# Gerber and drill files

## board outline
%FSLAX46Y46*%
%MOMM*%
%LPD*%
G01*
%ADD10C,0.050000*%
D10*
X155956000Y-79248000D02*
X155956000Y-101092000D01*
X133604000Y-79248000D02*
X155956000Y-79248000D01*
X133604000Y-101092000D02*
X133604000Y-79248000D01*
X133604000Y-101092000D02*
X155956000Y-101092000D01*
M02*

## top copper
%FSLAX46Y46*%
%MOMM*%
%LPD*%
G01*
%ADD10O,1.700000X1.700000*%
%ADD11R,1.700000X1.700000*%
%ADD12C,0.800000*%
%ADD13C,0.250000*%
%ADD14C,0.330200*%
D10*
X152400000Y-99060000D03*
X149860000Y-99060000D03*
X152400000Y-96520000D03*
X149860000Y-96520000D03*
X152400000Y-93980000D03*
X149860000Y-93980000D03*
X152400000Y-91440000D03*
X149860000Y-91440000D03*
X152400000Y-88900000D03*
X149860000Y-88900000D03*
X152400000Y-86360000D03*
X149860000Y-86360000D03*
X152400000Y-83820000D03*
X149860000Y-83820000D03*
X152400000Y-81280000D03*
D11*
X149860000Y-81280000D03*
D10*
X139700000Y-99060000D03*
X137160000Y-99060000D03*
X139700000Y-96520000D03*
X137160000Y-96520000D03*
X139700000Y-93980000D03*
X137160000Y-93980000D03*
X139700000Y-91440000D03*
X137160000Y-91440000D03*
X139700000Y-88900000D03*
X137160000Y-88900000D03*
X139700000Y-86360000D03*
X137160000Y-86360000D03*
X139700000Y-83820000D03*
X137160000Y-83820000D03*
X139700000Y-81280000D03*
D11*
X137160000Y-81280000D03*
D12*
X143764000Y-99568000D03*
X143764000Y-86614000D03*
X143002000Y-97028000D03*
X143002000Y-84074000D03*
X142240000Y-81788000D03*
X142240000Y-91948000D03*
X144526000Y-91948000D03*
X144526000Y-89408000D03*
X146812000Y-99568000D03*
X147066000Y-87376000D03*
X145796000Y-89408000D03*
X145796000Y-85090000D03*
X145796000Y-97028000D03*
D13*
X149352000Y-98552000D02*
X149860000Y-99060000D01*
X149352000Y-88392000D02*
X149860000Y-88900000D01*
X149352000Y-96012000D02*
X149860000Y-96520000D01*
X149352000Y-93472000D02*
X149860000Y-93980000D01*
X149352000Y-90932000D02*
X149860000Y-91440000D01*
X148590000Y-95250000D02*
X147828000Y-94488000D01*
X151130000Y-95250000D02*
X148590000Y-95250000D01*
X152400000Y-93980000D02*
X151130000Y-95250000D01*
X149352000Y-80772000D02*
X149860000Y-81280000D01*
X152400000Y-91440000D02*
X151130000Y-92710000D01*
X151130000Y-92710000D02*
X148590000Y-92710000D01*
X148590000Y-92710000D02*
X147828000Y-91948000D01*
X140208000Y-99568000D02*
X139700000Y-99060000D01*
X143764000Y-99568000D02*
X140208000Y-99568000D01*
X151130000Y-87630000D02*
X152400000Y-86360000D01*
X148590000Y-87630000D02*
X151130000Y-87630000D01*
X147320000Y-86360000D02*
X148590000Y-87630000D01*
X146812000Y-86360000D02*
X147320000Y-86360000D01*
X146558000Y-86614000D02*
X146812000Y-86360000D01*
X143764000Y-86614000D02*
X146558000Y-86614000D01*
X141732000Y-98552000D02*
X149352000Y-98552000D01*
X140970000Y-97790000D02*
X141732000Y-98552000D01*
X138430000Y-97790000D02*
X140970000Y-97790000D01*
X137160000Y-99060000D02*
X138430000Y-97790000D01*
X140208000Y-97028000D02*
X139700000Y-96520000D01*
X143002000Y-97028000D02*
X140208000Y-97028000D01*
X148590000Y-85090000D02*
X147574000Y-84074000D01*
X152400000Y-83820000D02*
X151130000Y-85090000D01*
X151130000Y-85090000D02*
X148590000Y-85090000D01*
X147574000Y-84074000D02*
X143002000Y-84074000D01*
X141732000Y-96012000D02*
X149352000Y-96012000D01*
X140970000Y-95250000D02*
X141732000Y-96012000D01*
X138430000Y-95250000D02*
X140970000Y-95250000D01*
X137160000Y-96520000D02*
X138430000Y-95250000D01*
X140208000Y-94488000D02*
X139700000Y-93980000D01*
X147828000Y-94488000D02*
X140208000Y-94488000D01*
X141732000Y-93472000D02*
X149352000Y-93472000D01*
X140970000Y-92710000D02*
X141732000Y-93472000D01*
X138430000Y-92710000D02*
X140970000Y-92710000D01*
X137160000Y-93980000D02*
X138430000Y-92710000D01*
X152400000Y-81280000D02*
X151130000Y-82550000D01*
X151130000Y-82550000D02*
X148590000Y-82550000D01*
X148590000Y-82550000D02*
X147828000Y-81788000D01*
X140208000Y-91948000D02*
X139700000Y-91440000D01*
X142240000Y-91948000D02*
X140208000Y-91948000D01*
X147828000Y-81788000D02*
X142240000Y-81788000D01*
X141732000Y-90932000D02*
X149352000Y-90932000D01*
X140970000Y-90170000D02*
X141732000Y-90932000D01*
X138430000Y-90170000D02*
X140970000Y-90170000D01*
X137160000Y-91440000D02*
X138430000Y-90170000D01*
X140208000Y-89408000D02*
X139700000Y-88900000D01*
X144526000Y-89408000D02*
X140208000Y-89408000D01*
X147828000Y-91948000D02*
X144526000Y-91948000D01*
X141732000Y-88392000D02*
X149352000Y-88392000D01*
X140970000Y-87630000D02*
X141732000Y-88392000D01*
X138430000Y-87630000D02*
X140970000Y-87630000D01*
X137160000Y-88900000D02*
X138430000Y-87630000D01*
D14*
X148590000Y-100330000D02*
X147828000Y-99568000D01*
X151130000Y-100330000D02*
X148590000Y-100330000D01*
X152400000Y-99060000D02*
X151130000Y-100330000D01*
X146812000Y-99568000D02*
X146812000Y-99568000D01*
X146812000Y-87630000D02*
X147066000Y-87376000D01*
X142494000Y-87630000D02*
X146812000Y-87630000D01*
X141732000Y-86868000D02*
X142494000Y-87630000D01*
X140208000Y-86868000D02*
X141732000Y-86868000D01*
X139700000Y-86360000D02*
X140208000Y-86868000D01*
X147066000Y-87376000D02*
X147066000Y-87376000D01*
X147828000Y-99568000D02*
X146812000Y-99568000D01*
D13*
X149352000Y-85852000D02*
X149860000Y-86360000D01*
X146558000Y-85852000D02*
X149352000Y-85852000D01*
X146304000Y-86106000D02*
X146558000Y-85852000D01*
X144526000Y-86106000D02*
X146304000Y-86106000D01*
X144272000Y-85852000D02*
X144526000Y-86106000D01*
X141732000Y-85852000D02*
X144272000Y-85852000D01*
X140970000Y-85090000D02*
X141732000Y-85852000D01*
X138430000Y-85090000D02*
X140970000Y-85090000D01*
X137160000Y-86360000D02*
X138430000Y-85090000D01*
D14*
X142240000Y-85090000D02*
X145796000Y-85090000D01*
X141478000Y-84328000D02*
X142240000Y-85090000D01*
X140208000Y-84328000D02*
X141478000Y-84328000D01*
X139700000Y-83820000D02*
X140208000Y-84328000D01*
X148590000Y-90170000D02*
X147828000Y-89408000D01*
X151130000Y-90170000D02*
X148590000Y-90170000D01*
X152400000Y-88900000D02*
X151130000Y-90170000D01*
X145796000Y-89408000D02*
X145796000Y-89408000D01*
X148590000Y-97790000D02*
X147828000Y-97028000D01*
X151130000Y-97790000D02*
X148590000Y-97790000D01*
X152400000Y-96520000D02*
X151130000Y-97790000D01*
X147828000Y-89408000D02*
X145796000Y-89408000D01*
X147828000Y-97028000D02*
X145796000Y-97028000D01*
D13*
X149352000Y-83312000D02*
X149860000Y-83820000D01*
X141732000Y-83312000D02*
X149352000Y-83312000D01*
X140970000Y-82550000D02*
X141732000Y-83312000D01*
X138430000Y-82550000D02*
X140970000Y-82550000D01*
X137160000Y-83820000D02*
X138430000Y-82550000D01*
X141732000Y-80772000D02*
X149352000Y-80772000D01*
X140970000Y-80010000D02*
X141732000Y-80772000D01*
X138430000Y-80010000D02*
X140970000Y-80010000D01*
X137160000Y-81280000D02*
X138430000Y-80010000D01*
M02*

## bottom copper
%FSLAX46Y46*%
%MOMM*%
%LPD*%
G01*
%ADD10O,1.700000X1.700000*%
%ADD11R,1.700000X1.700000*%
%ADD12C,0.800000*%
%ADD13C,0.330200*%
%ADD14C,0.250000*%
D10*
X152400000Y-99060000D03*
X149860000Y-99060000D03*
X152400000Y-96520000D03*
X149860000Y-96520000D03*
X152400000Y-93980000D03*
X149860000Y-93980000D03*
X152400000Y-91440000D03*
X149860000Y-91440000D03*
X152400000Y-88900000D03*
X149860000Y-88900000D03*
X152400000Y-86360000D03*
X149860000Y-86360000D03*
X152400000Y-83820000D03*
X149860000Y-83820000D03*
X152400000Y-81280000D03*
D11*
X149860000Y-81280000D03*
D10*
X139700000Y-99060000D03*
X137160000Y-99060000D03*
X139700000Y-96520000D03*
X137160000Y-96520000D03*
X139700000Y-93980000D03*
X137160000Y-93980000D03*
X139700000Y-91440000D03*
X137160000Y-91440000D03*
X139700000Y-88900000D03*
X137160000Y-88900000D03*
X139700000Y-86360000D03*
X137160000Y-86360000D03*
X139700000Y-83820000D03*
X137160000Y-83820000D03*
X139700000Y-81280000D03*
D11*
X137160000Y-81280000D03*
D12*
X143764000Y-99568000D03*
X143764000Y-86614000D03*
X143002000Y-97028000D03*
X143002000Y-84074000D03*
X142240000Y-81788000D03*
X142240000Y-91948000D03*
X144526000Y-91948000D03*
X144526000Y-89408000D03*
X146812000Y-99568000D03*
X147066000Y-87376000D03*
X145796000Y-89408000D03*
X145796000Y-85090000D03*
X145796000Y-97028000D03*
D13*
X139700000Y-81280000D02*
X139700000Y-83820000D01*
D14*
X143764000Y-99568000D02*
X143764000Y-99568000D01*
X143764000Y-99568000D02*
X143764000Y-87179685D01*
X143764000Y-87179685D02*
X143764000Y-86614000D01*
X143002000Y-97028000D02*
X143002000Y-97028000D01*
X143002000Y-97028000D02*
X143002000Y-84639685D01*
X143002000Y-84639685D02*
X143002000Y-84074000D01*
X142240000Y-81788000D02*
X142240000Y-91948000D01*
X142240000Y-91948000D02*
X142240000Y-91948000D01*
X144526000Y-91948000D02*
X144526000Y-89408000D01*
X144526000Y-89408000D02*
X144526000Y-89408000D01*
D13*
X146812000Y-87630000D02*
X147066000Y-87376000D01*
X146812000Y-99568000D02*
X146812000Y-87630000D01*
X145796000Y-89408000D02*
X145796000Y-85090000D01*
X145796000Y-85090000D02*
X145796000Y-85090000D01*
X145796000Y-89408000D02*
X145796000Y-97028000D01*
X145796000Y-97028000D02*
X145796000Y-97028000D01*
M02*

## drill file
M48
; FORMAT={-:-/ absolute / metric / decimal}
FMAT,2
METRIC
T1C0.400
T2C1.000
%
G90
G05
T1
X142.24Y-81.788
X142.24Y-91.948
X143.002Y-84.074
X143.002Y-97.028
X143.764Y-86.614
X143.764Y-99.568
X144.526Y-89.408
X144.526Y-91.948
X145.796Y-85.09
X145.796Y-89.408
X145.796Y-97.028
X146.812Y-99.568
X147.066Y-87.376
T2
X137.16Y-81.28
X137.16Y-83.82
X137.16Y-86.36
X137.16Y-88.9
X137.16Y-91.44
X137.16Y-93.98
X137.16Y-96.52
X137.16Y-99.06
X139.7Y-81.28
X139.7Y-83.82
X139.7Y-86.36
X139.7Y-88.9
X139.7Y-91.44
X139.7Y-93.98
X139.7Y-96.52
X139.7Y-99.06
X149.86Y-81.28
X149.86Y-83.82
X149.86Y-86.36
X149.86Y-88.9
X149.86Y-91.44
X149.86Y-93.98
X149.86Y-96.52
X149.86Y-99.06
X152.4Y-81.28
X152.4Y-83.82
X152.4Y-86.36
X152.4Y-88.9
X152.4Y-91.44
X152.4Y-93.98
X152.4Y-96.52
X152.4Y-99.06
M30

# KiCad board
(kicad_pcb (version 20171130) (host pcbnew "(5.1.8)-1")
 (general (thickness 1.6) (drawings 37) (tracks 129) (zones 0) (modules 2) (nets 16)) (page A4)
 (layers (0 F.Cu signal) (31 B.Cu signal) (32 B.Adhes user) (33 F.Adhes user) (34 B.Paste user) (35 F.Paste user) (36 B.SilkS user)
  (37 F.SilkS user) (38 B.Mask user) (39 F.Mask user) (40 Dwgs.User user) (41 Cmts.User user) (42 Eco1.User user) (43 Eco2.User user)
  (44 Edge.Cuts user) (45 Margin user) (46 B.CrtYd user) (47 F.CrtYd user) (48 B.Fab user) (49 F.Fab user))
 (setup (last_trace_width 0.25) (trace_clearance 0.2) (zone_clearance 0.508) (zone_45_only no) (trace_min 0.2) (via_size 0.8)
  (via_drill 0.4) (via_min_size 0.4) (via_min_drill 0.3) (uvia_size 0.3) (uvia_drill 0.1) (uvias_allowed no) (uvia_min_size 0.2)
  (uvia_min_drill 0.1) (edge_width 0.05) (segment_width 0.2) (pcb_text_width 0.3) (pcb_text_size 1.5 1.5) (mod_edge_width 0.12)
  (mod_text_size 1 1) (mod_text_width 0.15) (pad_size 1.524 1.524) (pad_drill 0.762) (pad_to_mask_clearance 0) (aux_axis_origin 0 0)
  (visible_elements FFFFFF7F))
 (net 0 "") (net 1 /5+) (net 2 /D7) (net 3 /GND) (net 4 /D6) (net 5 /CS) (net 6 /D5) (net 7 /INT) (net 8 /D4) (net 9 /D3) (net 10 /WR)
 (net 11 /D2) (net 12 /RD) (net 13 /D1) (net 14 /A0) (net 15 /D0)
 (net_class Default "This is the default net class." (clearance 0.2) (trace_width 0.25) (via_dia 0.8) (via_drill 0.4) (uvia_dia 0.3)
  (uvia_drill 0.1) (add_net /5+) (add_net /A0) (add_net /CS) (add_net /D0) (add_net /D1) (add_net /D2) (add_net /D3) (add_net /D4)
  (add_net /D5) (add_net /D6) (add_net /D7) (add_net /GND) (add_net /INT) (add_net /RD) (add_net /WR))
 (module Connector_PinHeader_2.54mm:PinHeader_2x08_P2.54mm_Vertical (layer F.Cu) (at 149.86 81.28)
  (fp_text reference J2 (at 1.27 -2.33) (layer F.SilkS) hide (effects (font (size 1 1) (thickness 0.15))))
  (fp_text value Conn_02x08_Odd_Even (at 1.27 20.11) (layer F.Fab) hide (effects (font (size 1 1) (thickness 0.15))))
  (pad 16 thru_hole oval (at 2.54 17.78) (size 1.7 1.7) (drill 1) (layers *.Cu *.Mask) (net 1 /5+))
  (pad 15 thru_hole oval (at 0 17.78) (size 1.7 1.7) (drill 1) (layers *.Cu *.Mask) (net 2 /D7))
  (pad 14 thru_hole oval (at 2.54 15.24) (size 1.7 1.7) (drill 1) (layers *.Cu *.Mask) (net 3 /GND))
  (pad 13 thru_hole oval (at 0 15.24) (size 1.7 1.7) (drill 1) (layers *.Cu *.Mask) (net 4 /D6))
  (pad 12 thru_hole oval (at 2.54 12.7) (size 1.7 1.7) (drill 1) (layers *.Cu *.Mask) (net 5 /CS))
  (pad 11 thru_hole oval (at 0 12.7) (size 1.7 1.7) (drill 1) (layers *.Cu *.Mask) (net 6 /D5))
  (pad 10 thru_hole oval (at 2.54 10.16) (size 1.7 1.7) (drill 1) (layers *.Cu *.Mask) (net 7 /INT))
  (pad 9 thru_hole oval (at 0 10.16) (size 1.7 1.7) (drill 1) (layers *.Cu *.Mask) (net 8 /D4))
  (pad 8 thru_hole oval (at 2.54 7.62) (size 1.7 1.7) (drill 1) (layers *.Cu *.Mask) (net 3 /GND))
  (pad 7 thru_hole oval (at 0 7.62) (size 1.7 1.7) (drill 1) (layers *.Cu *.Mask) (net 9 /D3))
  (pad 6 thru_hole oval (at 2.54 5.08) (size 1.7 1.7) (drill 1) (layers *.Cu *.Mask) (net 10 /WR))
  (pad 5 thru_hole oval (at 0 5.08) (size 1.7 1.7) (drill 1) (layers *.Cu *.Mask) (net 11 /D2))
  (pad 4 thru_hole oval (at 2.54 2.54) (size 1.7 1.7) (drill 1) (layers *.Cu *.Mask) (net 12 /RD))
  (pad 3 thru_hole oval (at 0 2.54) (size 1.7 1.7) (drill 1) (layers *.Cu *.Mask) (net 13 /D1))
  (pad 2 thru_hole oval (at 2.54 0) (size 1.7 1.7) (drill 1) (layers *.Cu *.Mask) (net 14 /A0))
  (pad 1 thru_hole rect (at 0 0) (size 1.7 1.7) (drill 1) (layers *.Cu *.Mask) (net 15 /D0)))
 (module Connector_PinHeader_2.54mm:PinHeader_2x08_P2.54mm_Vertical (layer F.Cu) (at 137.16 81.28)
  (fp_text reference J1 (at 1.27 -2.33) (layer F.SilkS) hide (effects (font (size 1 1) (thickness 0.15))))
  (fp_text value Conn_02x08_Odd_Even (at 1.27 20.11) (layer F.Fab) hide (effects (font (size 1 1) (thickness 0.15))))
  (pad 16 thru_hole oval (at 2.54 17.78) (size 1.7 1.7) (drill 1) (layers *.Cu *.Mask) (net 10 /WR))
  (pad 15 thru_hole oval (at 0 17.78) (size 1.7 1.7) (drill 1) (layers *.Cu *.Mask) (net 2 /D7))
  (pad 14 thru_hole oval (at 2.54 15.24) (size 1.7 1.7) (drill 1) (layers *.Cu *.Mask) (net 12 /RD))
  (pad 13 thru_hole oval (at 0 15.24) (size 1.7 1.7) (drill 1) (layers *.Cu *.Mask) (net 4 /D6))
  (pad 12 thru_hole oval (at 2.54 12.7) (size 1.7 1.7) (drill 1) (layers *.Cu *.Mask) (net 5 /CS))
  (pad 11 thru_hole oval (at 0 12.7) (size 1.7 1.7) (drill 1) (layers *.Cu *.Mask) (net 6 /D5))
  (pad 10 thru_hole oval (at 2.54 10.16) (size 1.7 1.7) (drill 1) (layers *.Cu *.Mask) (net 14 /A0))
  (pad 9 thru_hole oval (at 0 10.16) (size 1.7 1.7) (drill 1) (layers *.Cu *.Mask) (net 8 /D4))
  (pad 8 thru_hole oval (at 2.54 7.62) (size 1.7 1.7) (drill 1) (layers *.Cu *.Mask) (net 7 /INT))
  (pad 7 thru_hole oval (at 0 7.62) (size 1.7 1.7) (drill 1) (layers *.Cu *.Mask) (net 9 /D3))
  (pad 6 thru_hole oval (at 2.54 5.08) (size 1.7 1.7) (drill 1) (layers *.Cu *.Mask) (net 1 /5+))
  (pad 5 thru_hole oval (at 0 5.08) (size 1.7 1.7) (drill 1) (layers *.Cu *.Mask) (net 11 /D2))
  (pad 4 thru_hole oval (at 2.54 2.54) (size 1.7 1.7) (drill 1) (layers *.Cu *.Mask) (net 3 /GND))
  (pad 3 thru_hole oval (at 0 2.54) (size 1.7 1.7) (drill 1) (layers *.Cu *.Mask) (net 13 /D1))
  (pad 2 thru_hole oval (at 2.54 0) (size 1.7 1.7) (drill 1) (layers *.Cu *.Mask) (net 3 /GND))
  (pad 1 thru_hole rect (at 0 0) (size 1.7 1.7) (drill 1) (layers *.Cu *.Mask) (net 15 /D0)))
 (gr_line (start 155.956 79.248) (end 155.956 101.092) (layer Edge.Cuts) (width 0.05))
 (gr_line (start 133.604 79.248) (end 155.956 79.248) (layer Edge.Cuts) (width 0.05))
 (gr_line (start 133.604 101.092) (end 133.604 79.248) (layer Edge.Cuts) (width 0.05))
 (gr_line (start 133.604 101.092) (end 155.956 101.092) (layer Edge.Cuts) (width 0.05))
 (segment (start 149.352 98.552) (end 149.86 99.06) (width 0.25) (layer F.Cu) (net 2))
 (segment (start 149.352 88.392) (end 149.86 88.9) (width 0.25) (layer F.Cu) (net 9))
 (segment (start 149.352 96.012) (end 149.86 96.52) (width 0.25) (layer F.Cu) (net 4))
 (segment (start 149.352 93.472) (end 149.86 93.98) (width 0.25) (layer F.Cu) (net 6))
 (segment (start 149.352 90.932) (end 149.86 91.44) (width 0.25) (layer F.Cu) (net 8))
 (segment (start 148.59 95.25) (end 147.828 94.488) (width 0.25) (layer F.Cu) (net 5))
 (segment (start 151.13 95.25) (end 148.59 95.25) (width 0.25) (layer F.Cu) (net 5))
 (segment (start 152.4 93.98) (end 151.13 95.25) (width 0.25) (layer F.Cu) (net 5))
 (segment (start 149.352 80.772) (end 149.86 81.28) (width 0.25) (layer F.Cu) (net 15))
 (segment (start 139.7 81.28) (end 139.7 83.82) (width 0.3302) (layer B.Cu) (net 3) (status 30))
 (segment (start 152.4 91.44) (end 151.13 92.71) (width 0.25) (layer F.Cu) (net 7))
 (segment (start 151.13 92.71) (end 148.59 92.71) (width 0.25) (layer F.Cu) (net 7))
 (segment (start 148.59 92.71) (end 147.828 91.948) (width 0.25) (layer F.Cu) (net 7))
 (segment (start 143.764 99.568) (end 143.764 99.568) (width 0.25) (layer B.Cu) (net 10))
 (via (at 143.764 99.568) (size 0.8) (drill 0.4) (layers F.Cu B.Cu) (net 10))
 (segment (start 140.208 99.568) (end 139.7 99.06) (width 0.25) (layer F.Cu) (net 10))
 (segment (start 143.764 99.568) (end 140.208 99.568) (width 0.25) (layer F.Cu) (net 10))
 (via (at 143.764 86.614) (size 0.8) (drill 0.4) (layers F.Cu B.Cu) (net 10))
 (segment (start 143.764 99.568) (end 143.764 87.179685) (width 0.25) (layer B.Cu) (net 10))
 (segment (start 143.764 87.179685) (end 143.764 86.614) (width 0.25) (layer B.Cu) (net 10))
 (segment (start 151.13 87.63) (end 152.4 86.36) (width 0.25) (layer F.Cu) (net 10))
 (segment (start 148.59 87.63) (end 151.13 87.63) (width 0.25) (layer F.Cu) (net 10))
 (segment (start 147.32 86.36) (end 148.59 87.63) (width 0.25) (layer F.Cu) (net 10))
 (segment (start 146.812 86.36) (end 147.32 86.36) (width 0.25) (layer F.Cu) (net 10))
 (segment (start 146.558 86.614) (end 146.812 86.36) (width 0.25) (layer F.Cu) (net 10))
 (segment (start 143.764 86.614) (end 146.558 86.614) (width 0.25) (layer F.Cu) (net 10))
 (segment (start 141.732 98.552) (end 149.352 98.552) (width 0.25) (layer F.Cu) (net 2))
 (segment (start 140.97 97.79) (end 141.732 98.552) (width 0.25) (layer F.Cu) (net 2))
 (segment (start 138.43 97.79) (end 140.97 97.79) (width 0.25) (layer F.Cu) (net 2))
 (segment (start 137.16 99.06) (end 138.43 97.79) (width 0.25) (layer F.Cu) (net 2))
 (segment (start 143.002 97.028) (end 143.002 97.028) (width 0.25) (layer B.Cu) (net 12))
 (via (at 143.002 97.028) (size 0.8) (drill 0.4) (layers F.Cu B.Cu) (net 12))
 (segment (start 140.208 97.028) (end 139.7 96.52) (width 0.25) (layer F.Cu) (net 12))
 (segment (start 143.002 97.028) (end 140.208 97.028) (width 0.25) (layer F.Cu) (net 12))
 (via (at 143.002 84.074) (size 0.8) (drill 0.4) (layers F.Cu B.Cu) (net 12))
 (segment (start 148.59 85.09) (end 147.574 84.074) (width 0.25) (layer F.Cu) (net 12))
 (segment (start 152.4 83.82) (end 151.13 85.09) (width 0.25) (layer F.Cu) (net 12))
 (segment (start 151.13 85.09) (end 148.59 85.09) (width 0.25) (layer F.Cu) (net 12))
 (segment (start 143.002 97.028) (end 143.002 84.639685) (width 0.25) (layer B.Cu) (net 12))
 (segment (start 143.002 84.639685) (end 143.002 84.074) (width 0.25) (layer B.Cu) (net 12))
 (segment (start 147.574 84.074) (end 143.002 84.074) (width 0.25) (layer F.Cu) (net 12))
 (segment (start 141.732 96.012) (end 149.352 96.012) (width 0.25) (layer F.Cu) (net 4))
 (segment (start 140.97 95.25) (end 141.732 96.012) (width 0.25) (layer F.Cu) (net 4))
 (segment (start 138.43 95.25) (end 140.97 95.25) (width 0.25) (layer F.Cu) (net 4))
 (segment (start 137.16 96.52) (end 138.43 95.25) (width 0.25) (layer F.Cu) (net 4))
 (segment (start 140.208 94.488) (end 139.7 93.98) (width 0.25) (layer F.Cu) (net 5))
 (segment (start 147.828 94.488) (end 140.208 94.488) (width 0.25) (layer F.Cu) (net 5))
 (segment (start 141.732 93.472) (end 149.352 93.472) (width 0.25) (layer F.Cu) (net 6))
 (segment (start 140.97 92.71) (end 141.732 93.472) (width 0.25) (layer F.Cu) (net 6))
 (segment (start 138.43 92.71) (end 140.97 92.71) (width 0.25) (layer F.Cu) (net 6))
 (segment (start 137.16 93.98) (end 138.43 92.71) (width 0.25) (layer F.Cu) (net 6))
 (segment (start 152.4 81.28) (end 151.13 82.55) (width 0.25) (layer F.Cu) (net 14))
 (segment (start 151.13 82.55) (end 148.59 82.55) (width 0.25) (layer F.Cu) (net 14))
 (segment (start 148.59 82.55) (end 147.828 81.788) (width 0.25) (layer F.Cu) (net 14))
 (via (at 142.24 81.788) (size 0.8) (drill 0.4) (layers F.Cu B.Cu) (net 14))
 (segment (start 142.24 81.788) (end 142.24 91.948) (width 0.25) (layer B.Cu) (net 14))
 (segment (start 142.24 91.948) (end 142.24 91.948) (width 0.25) (layer B.Cu) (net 14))
 (via (at 142.24 91.948) (size 0.8) (drill 0.4) (layers F.Cu B.Cu) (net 14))
 (segment (start 140.208 91.948) (end 139.7 91.44) (width 0.25) (layer F.Cu) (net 14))
 (segment (start 142.24 91.948) (end 140.208 91.948) (width 0.25) (layer F.Cu) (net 14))
 (segment (start 147.828 81.788) (end 142.24 81.788) (width 0.25) (layer F.Cu) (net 14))
 (segment (start 141.732 90.932) (end 149.352 90.932) (width 0.25) (layer F.Cu) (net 8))
 (segment (start 140.97 90.17) (end 141.732 90.932) (width 0.25) (layer F.Cu) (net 8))
 (segment (start 138.43 90.17) (end 140.97 90.17) (width 0.25) (layer F.Cu) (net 8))
 (segment (start 137.16 91.44) (end 138.43 90.17) (width 0.25) (layer F.Cu) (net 8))
 (via (at 144.526 91.948) (size 0.8) (drill 0.4) (layers F.Cu B.Cu) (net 7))
 (segment (start 144.526 91.948) (end 144.526 89.408) (width 0.25) (layer B.Cu) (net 7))
 (segment (start 144.526 89.408) (end 144.526 89.408) (width 0.25) (layer B.Cu) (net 7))
 (via (at 144.526 89.408) (size 0.8) (drill 0.4) (layers F.Cu B.Cu) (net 7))
 (segment (start 140.208 89.408) (end 139.7 88.9) (width 0.25) (layer F.Cu) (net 7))
 (segment (start 144.526 89.408) (end 140.208 89.408) (width 0.25) (layer F.Cu) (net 7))
 (segment (start 147.828 91.948) (end 144.526 91.948) (width 0.25) (layer F.Cu) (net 7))
 (segment (start 141.732 88.392) (end 149.352 88.392) (width 0.25) (layer F.Cu) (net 9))
 (segment (start 140.97 87.63) (end 141.732 88.392) (width 0.25) (layer F.Cu) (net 9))
 (segment (start 138.43 87.63) (end 140.97 87.63) (width 0.25) (layer F.Cu) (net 9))
 (segment (start 137.16 88.9) (end 138.43 87.63) (width 0.25) (layer F.Cu) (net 9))
 (segment (start 148.59 100.33) (end 147.828 99.568) (width 0.3302) (layer F.Cu) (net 1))
 (segment (start 151.13 100.33) (end 148.59 100.33) (width 0.3302) (layer F.Cu) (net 1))
 (segment (start 152.4 99.06) (end 151.13 100.33) (width 0.3302) (layer F.Cu) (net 1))
 (segment (start 146.812 99.568) (end 146.812 99.568) (width 0.3302) (layer F.Cu) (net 1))
 (via (at 146.812 99.568) (size 0.8) (drill 0.4) (layers F.Cu B.Cu) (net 1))
 (segment (start 146.812 87.63) (end 147.066 87.376) (width 0.3302) (layer B.Cu) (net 1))
 (segment (start 146.812 99.568) (end 146.812 87.63) (width 0.3302) (layer B.Cu) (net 1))
 (segment (start 146.812 87.63) (end 147.066 87.376) (width 0.3302) (layer F.Cu) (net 1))
 (segment (start 142.494 87.63) (end 146.812 87.63) (width 0.3302) (layer F.Cu) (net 1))
 (segment (start 141.732 86.868) (end 142.494 87.63) (width 0.3302) (layer F.Cu) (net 1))
 (segment (start 140.208 86.868) (end 141.732 86.868) (width 0.3302) (layer F.Cu) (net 1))
 (segment (start 139.7 86.36) (end 140.208 86.868) (width 0.3302) (layer F.Cu) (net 1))
 (segment (start 147.066 87.376) (end 147.066 87.376) (width 0.3302) (layer F.Cu) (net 1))
 (via (at 147.066 87.376) (size 0.8) (drill 0.4) (layers F.Cu B.Cu) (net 1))
 (segment (start 147.828 99.568) (end 146.812 99.568) (width 0.3302) (layer F.Cu) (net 1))
 (segment (start 149.352 85.852) (end 149.86 86.36) (width 0.25) (layer F.Cu) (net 11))
 (segment (start 146.558 85.852) (end 149.352 85.852) (width 0.25) (layer F.Cu) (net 11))
 (segment (start 146.304 86.106) (end 146.558 85.852) (width 0.25) (layer F.Cu) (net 11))
 (segment (start 144.526 86.106) (end 146.304 86.106) (width 0.25) (layer F.Cu) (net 11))
 (segment (start 144.272 85.852) (end 144.526 86.106) (width 0.25) (layer F.Cu) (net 11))
 (segment (start 141.732 85.852) (end 144.272 85.852) (width 0.25) (layer F.Cu) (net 11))
 (segment (start 140.97 85.09) (end 141.732 85.852) (width 0.25) (layer F.Cu) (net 11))
 (segment (start 138.43 85.09) (end 140.97 85.09) (width 0.25) (layer F.Cu) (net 11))
 (segment (start 137.16 86.36) (end 138.43 85.09) (width 0.25) (layer F.Cu) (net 11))
 (segment (start 142.24 85.09) (end 145.796 85.09) (width 0.3302) (layer F.Cu) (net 3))
 (segment (start 141.478 84.328) (end 142.24 85.09) (width 0.3302) (layer F.Cu) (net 3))
 (segment (start 140.208 84.328) (end 141.478 84.328) (width 0.3302) (layer F.Cu) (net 3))
 (segment (start 139.7 83.82) (end 140.208 84.328) (width 0.3302) (layer F.Cu) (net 3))
 (segment (start 148.59 90.17) (end 147.828 89.408) (width 0.3302) (layer F.Cu) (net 3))
 (segment (start 151.13 90.17) (end 148.59 90.17) (width 0.3302) (layer F.Cu) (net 3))
 (segment (start 152.4 88.9) (end 151.13 90.17) (width 0.3302) (layer F.Cu) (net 3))
 (segment (start 145.796 89.408) (end 145.796 89.408) (width 0.3302) (layer F.Cu) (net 3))
 (via (at 145.796 89.408) (size 0.8) (drill 0.4) (layers F.Cu B.Cu) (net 3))
 (segment (start 145.796 89.408) (end 145.796 85.09) (width 0.3302) (layer B.Cu) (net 3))
 (segment (start 145.796 85.09) (end 145.796 85.09) (width 0.3302) (layer B.Cu) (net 3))
 (via (at 145.796 85.09) (size 0.8) (drill 0.4) (layers F.Cu B.Cu) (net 3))
 (segment (start 145.796 89.408) (end 145.796 97.028) (width 0.3302) (layer B.Cu) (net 3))
 (segment (start 148.59 97.79) (end 147.828 97.028) (width 0.3302) (layer F.Cu) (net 3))
 (segment (start 151.13 97.79) (end 148.59 97.79) (width 0.3302) (layer F.Cu) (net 3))
 (segment (start 152.4 96.52) (end 151.13 97.79) (width 0.3302) (layer F.Cu) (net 3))
 (segment (start 145.796 97.028) (end 145.796 97.028) (width 0.3302) (layer B.Cu) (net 3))
 (via (at 145.796 97.028) (size 0.8) (drill 0.4) (layers F.Cu B.Cu) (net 3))
 (segment (start 147.828 89.408) (end 145.796 89.408) (width 0.3302) (layer F.Cu) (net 3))
 (segment (start 147.828 97.028) (end 145.796 97.028) (width 0.3302) (layer F.Cu) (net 3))
 (segment (start 149.352 83.312) (end 149.86 83.82) (width 0.25) (layer F.Cu) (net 13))
 (segment (start 141.732 83.312) (end 149.352 83.312) (width 0.25) (layer F.Cu) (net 13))
 (segment (start 140.97 82.55) (end 141.732 83.312) (width 0.25) (layer F.Cu) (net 13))
 (segment (start 138.43 82.55) (end 140.97 82.55) (width 0.25) (layer F.Cu) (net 13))
 (segment (start 137.16 83.82) (end 138.43 82.55) (width 0.25) (layer F.Cu) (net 13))
 (segment (start 141.732 80.772) (end 149.352 80.772) (width 0.25) (layer F.Cu) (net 15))
 (segment (start 140.97 80.01) (end 141.732 80.772) (width 0.25) (layer F.Cu) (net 15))
 (segment (start 138.43 80.01) (end 140.97 80.01) (width 0.25) (layer F.Cu) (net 15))
 (segment (start 137.16 81.28) (end 138.43 80.01) (width 0.25) (layer F.Cu) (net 15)))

